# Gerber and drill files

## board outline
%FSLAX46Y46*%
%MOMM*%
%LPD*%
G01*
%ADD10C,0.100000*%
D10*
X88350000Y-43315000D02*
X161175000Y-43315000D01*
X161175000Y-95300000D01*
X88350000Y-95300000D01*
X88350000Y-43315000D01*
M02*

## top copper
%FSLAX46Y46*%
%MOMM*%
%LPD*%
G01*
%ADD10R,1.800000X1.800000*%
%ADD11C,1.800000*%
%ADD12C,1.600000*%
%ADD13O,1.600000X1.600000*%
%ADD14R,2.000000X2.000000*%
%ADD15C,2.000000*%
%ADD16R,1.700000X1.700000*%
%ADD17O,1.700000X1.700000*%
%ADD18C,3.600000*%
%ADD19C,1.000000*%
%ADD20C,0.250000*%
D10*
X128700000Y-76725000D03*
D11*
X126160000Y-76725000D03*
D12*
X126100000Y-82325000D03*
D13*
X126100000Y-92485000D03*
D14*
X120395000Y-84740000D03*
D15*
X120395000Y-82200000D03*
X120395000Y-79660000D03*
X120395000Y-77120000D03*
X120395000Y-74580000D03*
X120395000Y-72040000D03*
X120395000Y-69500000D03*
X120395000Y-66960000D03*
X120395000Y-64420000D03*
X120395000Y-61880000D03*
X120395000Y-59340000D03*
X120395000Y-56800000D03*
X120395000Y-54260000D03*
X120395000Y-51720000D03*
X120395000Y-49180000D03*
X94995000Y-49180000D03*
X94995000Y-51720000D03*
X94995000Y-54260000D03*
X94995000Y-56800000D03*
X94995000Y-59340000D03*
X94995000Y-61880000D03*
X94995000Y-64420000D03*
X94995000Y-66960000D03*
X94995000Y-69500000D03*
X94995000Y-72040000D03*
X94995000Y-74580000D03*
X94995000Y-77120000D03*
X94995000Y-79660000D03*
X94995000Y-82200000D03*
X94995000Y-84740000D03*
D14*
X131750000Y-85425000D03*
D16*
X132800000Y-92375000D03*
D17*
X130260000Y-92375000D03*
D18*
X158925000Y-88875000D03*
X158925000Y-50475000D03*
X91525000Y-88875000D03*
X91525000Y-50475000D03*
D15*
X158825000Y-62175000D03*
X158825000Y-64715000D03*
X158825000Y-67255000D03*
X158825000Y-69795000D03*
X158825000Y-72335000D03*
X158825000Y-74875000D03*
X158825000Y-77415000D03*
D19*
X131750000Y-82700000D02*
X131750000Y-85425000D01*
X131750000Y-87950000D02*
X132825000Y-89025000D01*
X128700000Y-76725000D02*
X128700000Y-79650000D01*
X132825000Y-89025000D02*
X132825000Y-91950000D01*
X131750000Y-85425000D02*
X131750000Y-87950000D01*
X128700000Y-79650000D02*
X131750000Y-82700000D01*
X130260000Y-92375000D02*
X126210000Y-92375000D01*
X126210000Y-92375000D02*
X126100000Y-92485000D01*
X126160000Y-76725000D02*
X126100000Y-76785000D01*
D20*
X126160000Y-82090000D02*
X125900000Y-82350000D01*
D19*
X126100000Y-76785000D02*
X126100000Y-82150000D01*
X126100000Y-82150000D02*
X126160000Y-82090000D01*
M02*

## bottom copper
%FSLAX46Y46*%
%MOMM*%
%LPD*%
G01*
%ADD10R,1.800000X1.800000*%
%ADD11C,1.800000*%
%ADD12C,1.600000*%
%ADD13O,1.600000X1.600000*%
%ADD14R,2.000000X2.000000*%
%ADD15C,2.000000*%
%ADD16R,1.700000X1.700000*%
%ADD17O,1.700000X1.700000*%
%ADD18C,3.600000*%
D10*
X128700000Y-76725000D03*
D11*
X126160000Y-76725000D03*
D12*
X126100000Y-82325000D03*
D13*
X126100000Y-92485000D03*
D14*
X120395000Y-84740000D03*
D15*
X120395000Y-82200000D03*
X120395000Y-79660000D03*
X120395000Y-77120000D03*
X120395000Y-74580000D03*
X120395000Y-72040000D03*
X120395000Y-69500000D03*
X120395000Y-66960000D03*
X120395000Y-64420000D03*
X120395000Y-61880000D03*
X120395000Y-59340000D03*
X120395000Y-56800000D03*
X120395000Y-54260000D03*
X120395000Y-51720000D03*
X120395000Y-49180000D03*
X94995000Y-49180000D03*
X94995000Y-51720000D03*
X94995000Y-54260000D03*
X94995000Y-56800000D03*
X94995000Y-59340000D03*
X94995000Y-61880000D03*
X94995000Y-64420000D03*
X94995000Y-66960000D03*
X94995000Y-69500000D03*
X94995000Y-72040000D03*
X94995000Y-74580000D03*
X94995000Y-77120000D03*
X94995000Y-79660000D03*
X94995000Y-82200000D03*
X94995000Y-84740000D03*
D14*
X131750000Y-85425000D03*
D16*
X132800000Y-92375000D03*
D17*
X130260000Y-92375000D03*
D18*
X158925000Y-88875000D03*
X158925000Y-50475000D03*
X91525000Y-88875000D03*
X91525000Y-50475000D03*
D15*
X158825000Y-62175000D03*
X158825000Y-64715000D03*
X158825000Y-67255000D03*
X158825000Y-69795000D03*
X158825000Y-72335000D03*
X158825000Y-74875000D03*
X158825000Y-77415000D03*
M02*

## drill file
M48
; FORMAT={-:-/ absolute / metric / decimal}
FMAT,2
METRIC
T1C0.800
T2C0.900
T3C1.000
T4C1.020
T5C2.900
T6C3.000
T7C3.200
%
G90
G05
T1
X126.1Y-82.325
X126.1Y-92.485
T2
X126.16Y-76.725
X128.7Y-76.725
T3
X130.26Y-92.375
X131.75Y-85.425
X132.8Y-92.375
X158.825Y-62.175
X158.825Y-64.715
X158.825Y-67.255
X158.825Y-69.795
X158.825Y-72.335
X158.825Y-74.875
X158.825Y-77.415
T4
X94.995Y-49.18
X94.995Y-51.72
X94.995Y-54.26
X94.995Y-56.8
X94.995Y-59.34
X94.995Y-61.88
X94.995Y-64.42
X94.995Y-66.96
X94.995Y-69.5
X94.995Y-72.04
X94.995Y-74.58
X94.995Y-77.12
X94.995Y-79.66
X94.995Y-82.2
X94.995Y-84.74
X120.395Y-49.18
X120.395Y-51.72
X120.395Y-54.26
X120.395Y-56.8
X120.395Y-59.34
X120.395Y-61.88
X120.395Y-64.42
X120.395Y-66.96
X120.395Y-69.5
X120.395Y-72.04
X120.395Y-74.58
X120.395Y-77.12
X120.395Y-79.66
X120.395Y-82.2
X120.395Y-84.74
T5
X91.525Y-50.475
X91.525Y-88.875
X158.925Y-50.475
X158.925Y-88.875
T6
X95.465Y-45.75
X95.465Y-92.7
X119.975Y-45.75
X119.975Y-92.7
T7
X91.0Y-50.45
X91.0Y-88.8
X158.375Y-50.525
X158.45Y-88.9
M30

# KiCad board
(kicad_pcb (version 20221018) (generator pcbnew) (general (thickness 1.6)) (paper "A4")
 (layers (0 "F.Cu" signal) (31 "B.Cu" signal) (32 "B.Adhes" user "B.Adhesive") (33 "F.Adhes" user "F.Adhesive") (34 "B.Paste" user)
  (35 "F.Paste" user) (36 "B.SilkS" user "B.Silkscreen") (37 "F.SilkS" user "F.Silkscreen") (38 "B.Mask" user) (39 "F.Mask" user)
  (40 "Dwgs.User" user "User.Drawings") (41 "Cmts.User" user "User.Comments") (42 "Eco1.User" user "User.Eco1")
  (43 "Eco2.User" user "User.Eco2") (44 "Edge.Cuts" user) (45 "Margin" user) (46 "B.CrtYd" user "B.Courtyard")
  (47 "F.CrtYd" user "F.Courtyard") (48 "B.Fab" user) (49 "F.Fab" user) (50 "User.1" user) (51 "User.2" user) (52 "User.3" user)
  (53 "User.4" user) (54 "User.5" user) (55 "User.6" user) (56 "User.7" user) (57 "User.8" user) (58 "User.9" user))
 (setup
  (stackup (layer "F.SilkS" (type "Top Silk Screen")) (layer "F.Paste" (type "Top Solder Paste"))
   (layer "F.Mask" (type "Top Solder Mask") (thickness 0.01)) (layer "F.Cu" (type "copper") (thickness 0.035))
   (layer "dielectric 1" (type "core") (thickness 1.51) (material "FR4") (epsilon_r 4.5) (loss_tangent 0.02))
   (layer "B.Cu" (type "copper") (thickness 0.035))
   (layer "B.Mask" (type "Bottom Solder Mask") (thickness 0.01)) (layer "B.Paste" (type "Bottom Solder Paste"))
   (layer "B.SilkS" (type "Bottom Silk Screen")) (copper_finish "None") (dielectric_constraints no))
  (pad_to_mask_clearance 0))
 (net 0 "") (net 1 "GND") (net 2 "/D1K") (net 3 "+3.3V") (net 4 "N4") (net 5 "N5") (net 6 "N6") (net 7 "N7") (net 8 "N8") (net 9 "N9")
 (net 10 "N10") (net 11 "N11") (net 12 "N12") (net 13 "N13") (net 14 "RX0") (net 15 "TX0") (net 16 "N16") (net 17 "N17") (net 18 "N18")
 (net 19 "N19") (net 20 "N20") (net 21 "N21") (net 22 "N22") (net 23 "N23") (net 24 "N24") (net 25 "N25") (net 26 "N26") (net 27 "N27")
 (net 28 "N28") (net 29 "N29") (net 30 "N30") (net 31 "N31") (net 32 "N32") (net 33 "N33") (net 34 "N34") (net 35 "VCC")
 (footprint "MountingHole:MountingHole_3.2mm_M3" (layer "F.Cu") (at 158.45 88.9)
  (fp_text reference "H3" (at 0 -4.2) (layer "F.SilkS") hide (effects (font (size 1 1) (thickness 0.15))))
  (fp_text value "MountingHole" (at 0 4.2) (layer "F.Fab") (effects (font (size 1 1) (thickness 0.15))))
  (pad "" np_thru_hole circle (at 0 0) (size 3.2 3.2) (drill 3.2) (layers "*.Cu" "*.Mask")))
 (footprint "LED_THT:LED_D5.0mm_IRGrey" (layer "F.Cu") (at 128.7 76.725 180)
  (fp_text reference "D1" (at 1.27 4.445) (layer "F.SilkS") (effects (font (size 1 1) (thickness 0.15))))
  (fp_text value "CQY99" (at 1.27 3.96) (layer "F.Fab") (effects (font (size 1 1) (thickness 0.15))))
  (pad "1" thru_hole rect (at 0 0 180) (size 1.8 1.8) (drill 0.9) (layers "*.Cu" "*.Mask") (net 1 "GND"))
  (pad "2" thru_hole circle (at 2.54 0 180) (size 1.8 1.8) (drill 0.9) (layers "*.Cu" "*.Mask") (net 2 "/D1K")))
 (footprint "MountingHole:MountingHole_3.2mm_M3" (layer "F.Cu") (at 91 50.45)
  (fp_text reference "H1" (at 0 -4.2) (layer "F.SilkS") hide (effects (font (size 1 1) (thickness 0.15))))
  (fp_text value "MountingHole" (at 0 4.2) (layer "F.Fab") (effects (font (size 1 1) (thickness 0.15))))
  (pad "" np_thru_hole circle (at 0 0) (size 3.2 3.2) (drill 3.2) (layers "*.Cu" "*.Mask")))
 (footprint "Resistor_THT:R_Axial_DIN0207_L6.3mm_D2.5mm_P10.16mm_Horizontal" (layer "F.Cu") (at 126.1 82.325 -90)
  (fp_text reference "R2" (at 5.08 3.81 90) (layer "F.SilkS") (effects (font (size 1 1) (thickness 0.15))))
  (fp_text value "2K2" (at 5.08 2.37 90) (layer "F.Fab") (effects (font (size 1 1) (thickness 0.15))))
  (pad "1" thru_hole circle (at 0 0 270) (size 1.6 1.6) (drill 0.8) (layers "*.Cu" "*.Mask") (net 2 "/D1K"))
  (pad "2" thru_hole oval (at 10.16 0 270) (size 1.6 1.6) (drill 0.8) (layers "*.Cu" "*.Mask") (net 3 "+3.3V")))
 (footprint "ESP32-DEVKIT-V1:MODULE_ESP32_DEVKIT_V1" (layer "F.Cu") (at 107.695 69.225 180)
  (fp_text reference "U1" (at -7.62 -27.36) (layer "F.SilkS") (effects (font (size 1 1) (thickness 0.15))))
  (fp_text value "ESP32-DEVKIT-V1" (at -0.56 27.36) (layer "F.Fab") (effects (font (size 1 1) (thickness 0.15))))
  (pad "" np_thru_hole circle (at -12.28 -23.475 180) (size 3 3) (drill 3) (layers "*.Cu" "*.Mask"))
  (pad "" np_thru_hole circle (at -12.28 23.475 180) (size 3 3) (drill 3) (layers "*.Cu" "*.Mask"))
  (pad "" np_thru_hole circle (at 12.23 -23.475 180) (size 3 3) (drill 3) (layers "*.Cu" "*.Mask"))
  (pad "" np_thru_hole circle (at 12.23 23.475 180) (size 3 3) (drill 3) (layers "*.Cu" "*.Mask"))
  (pad "1" thru_hole rect (at -12.7 -15.515 180) (size 2 2) (drill 1.02) (layers "*.Cu" "*.Mask") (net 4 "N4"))
  (pad "2" thru_hole circle (at -12.7 -12.975 180) (size 2 2) (drill 1.02) (layers "*.Cu" "*.Mask") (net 1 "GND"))
  (pad "3" thru_hole circle (at -12.7 -10.435 180) (size 2 2) (drill 1.02) (layers "*.Cu" "*.Mask") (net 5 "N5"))
  (pad "4" thru_hole circle (at -12.7 -7.895 180) (size 2 2) (drill 1.02) (layers "*.Cu" "*.Mask") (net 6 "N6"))
  (pad "5" thru_hole circle (at -12.7 -5.355 180) (size 2 2) (drill 1.02) (layers "*.Cu" "*.Mask") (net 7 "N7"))
  (pad "6" thru_hole circle (at -12.7 -2.815 180) (size 2 2) (drill 1.02) (layers "*.Cu" "*.Mask") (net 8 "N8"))
  (pad "7" thru_hole circle (at -12.7 -0.275 180) (size 2 2) (drill 1.02) (layers "*.Cu" "*.Mask") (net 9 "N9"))
  (pad "8" thru_hole circle (at -12.7 2.265 180) (size 2 2) (drill 1.02) (layers "*.Cu" "*.Mask") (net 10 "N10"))
  (pad "9" thru_hole circle (at -12.7 4.805 180) (size 2 2) (drill 1.02) (layers "*.Cu" "*.Mask") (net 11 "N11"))
  (pad "10" thru_hole circle (at -12.7 7.345 180) (size 2 2) (drill 1.02) (layers "*.Cu" "*.Mask") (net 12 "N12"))
  (pad "11" thru_hole circle (at -12.7 9.885 180) (size 2 2) (drill 1.02) (layers "*.Cu" "*.Mask") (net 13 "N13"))
  (pad "12" thru_hole circle (at -12.7 12.425 180) (size 2 2) (drill 1.02) (layers "*.Cu" "*.Mask") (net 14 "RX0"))
  (pad "13" thru_hole circle (at -12.7 14.965 180) (size 2 2) (drill 1.02) (layers "*.Cu" "*.Mask") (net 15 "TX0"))
  (pad "14" thru_hole circle (at -12.7 17.505 180) (size 2 2) (drill 1.02) (layers "*.Cu" "*.Mask") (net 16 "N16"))
  (pad "15" thru_hole circle (at -12.7 20.045 180) (size 2 2) (drill 1.02) (layers "*.Cu" "*.Mask") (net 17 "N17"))
  (pad "16" thru_hole circle (at 12.7 20.045 180) (size 2 2) (drill 1.02) (layers "*.Cu" "*.Mask") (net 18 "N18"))
  (pad "17" thru_hole circle (at 12.7 17.505 180) (size 2 2) (drill 1.02) (layers "*.Cu" "*.Mask") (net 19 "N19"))
  (pad "18" thru_hole circle (at 12.7 14.965 180) (size 2 2) (drill 1.02) (layers "*.Cu" "*.Mask") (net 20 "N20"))
  (pad "19" thru_hole circle (at 12.7 12.425 180) (size 2 2) (drill 1.02) (layers "*.Cu" "*.Mask") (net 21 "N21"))
  (pad "20" thru_hole circle (at 12.7 9.885 180) (size 2 2) (drill 1.02) (layers "*.Cu" "*.Mask") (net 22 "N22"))
  (pad "21" thru_hole circle (at 12.7 7.345 180) (size 2 2) (drill 1.02) (layers "*.Cu" "*.Mask") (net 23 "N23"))
  (pad "22" thru_hole circle (at 12.7 4.805 180) (size 2 2) (drill 1.02) (layers "*.Cu" "*.Mask") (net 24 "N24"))
  (pad "23" thru_hole circle (at 12.7 2.265 180) (size 2 2) (drill 1.02) (layers "*.Cu" "*.Mask") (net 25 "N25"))
  (pad "24" thru_hole circle (at 12.7 -0.275 180) (size 2 2) (drill 1.02) (layers "*.Cu" "*.Mask") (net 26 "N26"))
  (pad "25" thru_hole circle (at 12.7 -2.815 180) (size 2 2) (drill 1.02) (layers "*.Cu" "*.Mask") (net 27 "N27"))
  (pad "26" thru_hole circle (at 12.7 -5.355 180) (size 2 2) (drill 1.02) (layers "*.Cu" "*.Mask") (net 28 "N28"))
  (pad "27" thru_hole circle (at 12.7 -7.895 180) (size 2 2) (drill 1.02) (layers "*.Cu" "*.Mask") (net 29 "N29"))
  (pad "28" thru_hole circle (at 12.7 -10.435 180) (size 2 2) (drill 1.02) (layers "*.Cu" "*.Mask") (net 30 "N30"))
  (pad "29" thru_hole circle (at 12.7 -12.975 180) (size 2 2) (drill 1.02) (layers "*.Cu" "*.Mask") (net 1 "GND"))
  (pad "30" thru_hole circle (at 12.7 -15.515 180) (size 2 2) (drill 1.02) (layers "*.Cu" "*.Mask") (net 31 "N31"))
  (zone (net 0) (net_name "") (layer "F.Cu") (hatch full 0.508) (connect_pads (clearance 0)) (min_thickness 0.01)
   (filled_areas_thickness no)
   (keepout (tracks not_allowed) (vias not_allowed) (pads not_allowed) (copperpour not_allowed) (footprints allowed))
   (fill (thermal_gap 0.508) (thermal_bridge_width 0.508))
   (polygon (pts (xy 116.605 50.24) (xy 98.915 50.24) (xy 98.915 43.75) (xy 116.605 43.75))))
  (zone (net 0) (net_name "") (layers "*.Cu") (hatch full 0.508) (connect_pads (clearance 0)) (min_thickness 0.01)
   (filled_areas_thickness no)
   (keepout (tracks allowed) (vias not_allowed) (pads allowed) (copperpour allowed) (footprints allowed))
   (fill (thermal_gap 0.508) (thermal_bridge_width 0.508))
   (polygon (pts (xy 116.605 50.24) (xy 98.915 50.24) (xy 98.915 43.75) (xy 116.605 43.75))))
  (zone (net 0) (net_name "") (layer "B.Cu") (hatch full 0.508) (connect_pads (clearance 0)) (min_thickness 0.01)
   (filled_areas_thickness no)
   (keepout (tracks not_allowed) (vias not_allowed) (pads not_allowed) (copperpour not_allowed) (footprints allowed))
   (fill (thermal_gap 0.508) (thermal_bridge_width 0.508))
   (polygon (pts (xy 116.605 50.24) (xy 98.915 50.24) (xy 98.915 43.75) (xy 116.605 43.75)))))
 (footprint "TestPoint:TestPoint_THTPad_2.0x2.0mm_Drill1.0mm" (layer "F.Cu") (at 131.75 85.425)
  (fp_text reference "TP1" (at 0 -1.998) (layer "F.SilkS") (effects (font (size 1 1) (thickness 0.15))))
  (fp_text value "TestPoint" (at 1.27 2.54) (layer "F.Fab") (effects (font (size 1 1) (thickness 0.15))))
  (pad "1" thru_hole rect (at 0 0) (size 2 2) (drill 1) (layers "*.Cu" "*.Mask") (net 1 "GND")))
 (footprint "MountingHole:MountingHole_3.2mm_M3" (layer "F.Cu") (at 91 88.8)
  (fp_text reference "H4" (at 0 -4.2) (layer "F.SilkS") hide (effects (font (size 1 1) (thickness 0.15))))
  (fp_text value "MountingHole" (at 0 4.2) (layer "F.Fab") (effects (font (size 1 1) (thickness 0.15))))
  (pad "" np_thru_hole circle (at 0 0) (size 3.2 3.2) (drill 3.2) (layers "*.Cu" "*.Mask")))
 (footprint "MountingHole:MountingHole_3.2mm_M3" (layer "F.Cu") (at 158.375 50.525)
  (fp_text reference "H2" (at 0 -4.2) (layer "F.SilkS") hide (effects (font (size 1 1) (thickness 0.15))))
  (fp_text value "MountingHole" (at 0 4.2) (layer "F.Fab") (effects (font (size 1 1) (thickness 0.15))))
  (pad "" np_thru_hole circle (at 0 0) (size 3.2 3.2) (drill 3.2) (layers "*.Cu" "*.Mask")))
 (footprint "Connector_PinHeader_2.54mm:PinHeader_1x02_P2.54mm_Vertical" (layer "F.Cu") (at 132.8 92.375 -90)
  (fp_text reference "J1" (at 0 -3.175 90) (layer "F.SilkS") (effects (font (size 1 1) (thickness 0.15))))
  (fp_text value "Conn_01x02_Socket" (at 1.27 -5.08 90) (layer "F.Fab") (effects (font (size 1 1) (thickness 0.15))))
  (pad "1" thru_hole rect (at 0 0 270) (size 1.7 1.7) (drill 1) (layers "*.Cu" "*.Mask") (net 1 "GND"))
  (pad "2" thru_hole oval (at 0 2.54 270) (size 1.7 1.7) (drill 1) (layers "*.Cu" "*.Mask") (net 3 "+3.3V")))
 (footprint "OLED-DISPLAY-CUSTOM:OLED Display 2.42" (layer "B.Cu") (at 161.225 48.175 180)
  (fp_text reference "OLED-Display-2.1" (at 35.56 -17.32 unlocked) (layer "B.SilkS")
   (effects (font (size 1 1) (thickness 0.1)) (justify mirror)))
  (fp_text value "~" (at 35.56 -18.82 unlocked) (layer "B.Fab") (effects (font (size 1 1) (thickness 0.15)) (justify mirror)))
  (pad "" np_thru_hole circle (at 2.3 -40.7 180) (size 3.6 3.6) (drill 2.9) (layers "F&B.Cu" "*.Mask"))
  (pad "" np_thru_hole circle (at 2.3 -2.3 180) (size 3.6 3.6) (drill 2.9) (layers "F&B.Cu" "*.Mask"))
  (pad "" np_thru_hole circle (at 69.7 -40.7 180) (size 3.6 3.6) (drill 2.9) (layers "F&B.Cu" "*.Mask"))
  (pad "" np_thru_hole circle (at 69.7 -2.3 180) (size 3.6 3.6) (drill 2.9) (layers "F&B.Cu" "*.Mask"))
  (pad "1" thru_hole circle (at 2.4 -14 180) (size 2 2) (drill 1) (layers "*.Cu" "*.Mask") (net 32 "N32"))
  (pad "2" thru_hole circle (at 2.4 -16.54 180) (size 2 2) (drill 1) (layers "*.Cu" "*.Mask") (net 15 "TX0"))
  (pad "3" thru_hole circle (at 2.4 -19.08 180) (size 2 2) (drill 1) (layers "*.Cu" "*.Mask") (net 14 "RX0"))
  (pad "4" thru_hole circle (at 2.4 -21.62 180) (size 2 2) (drill 1) (layers "*.Cu" "*.Mask") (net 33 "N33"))
  (pad "5" thru_hole circle (at 2.4 -24.16 180) (size 2 2) (drill 1) (layers "*.Cu" "*.Mask") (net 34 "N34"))
  (pad "6" thru_hole circle (at 2.4 -26.7 180) (size 2 2) (drill 1) (layers "*.Cu" "*.Mask") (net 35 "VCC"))
  (pad "7" thru_hole circle (at 2.4 -29.24 180) (size 2 2) (drill 1) (layers "*.Cu" "*.Mask") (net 1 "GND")))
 (gr_rect (start 88.35 43.315) (end 161.175 95.3) (stroke (width 0.1) (type default)) (fill none) (layer "Edge.Cuts"))
 (segment (start 131.75 82.7) (end 131.75 85.425) (width 1) (layer "F.Cu") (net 1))
 (segment (start 131.75 87.95) (end 132.825 89.025) (width 1) (layer "F.Cu") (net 1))
 (segment (start 128.7 76.725) (end 128.7 79.65) (width 1) (layer "F.Cu") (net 1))
 (segment (start 132.825 89.025) (end 132.825 91.95) (width 1) (layer "F.Cu") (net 1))
 (segment (start 131.75 85.425) (end 131.75 87.95) (width 1) (layer "F.Cu") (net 1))
 (segment (start 128.7 79.65) (end 131.75 82.7) (width 1) (layer "F.Cu") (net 1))
 (segment (start 130.26 92.375) (end 126.21 92.375) (width 1) (layer "F.Cu") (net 3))
 (segment (start 126.21 92.375) (end 126.1 92.485) (width 1) (layer "F.Cu") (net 3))
 (segment (start 126.16 76.725) (end 126.1 76.785) (width 1) (layer "F.Cu") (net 2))
 (segment (start 126.16 82.09) (end 125.9 82.35) (width 0.25) (layer "F.Cu") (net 2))
 (segment (start 126.1 76.785) (end 126.1 82.15) (width 1) (layer "F.Cu") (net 2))
 (segment (start 126.1 82.15) (end 126.16 82.09) (width 1) (layer "F.Cu") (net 2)))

